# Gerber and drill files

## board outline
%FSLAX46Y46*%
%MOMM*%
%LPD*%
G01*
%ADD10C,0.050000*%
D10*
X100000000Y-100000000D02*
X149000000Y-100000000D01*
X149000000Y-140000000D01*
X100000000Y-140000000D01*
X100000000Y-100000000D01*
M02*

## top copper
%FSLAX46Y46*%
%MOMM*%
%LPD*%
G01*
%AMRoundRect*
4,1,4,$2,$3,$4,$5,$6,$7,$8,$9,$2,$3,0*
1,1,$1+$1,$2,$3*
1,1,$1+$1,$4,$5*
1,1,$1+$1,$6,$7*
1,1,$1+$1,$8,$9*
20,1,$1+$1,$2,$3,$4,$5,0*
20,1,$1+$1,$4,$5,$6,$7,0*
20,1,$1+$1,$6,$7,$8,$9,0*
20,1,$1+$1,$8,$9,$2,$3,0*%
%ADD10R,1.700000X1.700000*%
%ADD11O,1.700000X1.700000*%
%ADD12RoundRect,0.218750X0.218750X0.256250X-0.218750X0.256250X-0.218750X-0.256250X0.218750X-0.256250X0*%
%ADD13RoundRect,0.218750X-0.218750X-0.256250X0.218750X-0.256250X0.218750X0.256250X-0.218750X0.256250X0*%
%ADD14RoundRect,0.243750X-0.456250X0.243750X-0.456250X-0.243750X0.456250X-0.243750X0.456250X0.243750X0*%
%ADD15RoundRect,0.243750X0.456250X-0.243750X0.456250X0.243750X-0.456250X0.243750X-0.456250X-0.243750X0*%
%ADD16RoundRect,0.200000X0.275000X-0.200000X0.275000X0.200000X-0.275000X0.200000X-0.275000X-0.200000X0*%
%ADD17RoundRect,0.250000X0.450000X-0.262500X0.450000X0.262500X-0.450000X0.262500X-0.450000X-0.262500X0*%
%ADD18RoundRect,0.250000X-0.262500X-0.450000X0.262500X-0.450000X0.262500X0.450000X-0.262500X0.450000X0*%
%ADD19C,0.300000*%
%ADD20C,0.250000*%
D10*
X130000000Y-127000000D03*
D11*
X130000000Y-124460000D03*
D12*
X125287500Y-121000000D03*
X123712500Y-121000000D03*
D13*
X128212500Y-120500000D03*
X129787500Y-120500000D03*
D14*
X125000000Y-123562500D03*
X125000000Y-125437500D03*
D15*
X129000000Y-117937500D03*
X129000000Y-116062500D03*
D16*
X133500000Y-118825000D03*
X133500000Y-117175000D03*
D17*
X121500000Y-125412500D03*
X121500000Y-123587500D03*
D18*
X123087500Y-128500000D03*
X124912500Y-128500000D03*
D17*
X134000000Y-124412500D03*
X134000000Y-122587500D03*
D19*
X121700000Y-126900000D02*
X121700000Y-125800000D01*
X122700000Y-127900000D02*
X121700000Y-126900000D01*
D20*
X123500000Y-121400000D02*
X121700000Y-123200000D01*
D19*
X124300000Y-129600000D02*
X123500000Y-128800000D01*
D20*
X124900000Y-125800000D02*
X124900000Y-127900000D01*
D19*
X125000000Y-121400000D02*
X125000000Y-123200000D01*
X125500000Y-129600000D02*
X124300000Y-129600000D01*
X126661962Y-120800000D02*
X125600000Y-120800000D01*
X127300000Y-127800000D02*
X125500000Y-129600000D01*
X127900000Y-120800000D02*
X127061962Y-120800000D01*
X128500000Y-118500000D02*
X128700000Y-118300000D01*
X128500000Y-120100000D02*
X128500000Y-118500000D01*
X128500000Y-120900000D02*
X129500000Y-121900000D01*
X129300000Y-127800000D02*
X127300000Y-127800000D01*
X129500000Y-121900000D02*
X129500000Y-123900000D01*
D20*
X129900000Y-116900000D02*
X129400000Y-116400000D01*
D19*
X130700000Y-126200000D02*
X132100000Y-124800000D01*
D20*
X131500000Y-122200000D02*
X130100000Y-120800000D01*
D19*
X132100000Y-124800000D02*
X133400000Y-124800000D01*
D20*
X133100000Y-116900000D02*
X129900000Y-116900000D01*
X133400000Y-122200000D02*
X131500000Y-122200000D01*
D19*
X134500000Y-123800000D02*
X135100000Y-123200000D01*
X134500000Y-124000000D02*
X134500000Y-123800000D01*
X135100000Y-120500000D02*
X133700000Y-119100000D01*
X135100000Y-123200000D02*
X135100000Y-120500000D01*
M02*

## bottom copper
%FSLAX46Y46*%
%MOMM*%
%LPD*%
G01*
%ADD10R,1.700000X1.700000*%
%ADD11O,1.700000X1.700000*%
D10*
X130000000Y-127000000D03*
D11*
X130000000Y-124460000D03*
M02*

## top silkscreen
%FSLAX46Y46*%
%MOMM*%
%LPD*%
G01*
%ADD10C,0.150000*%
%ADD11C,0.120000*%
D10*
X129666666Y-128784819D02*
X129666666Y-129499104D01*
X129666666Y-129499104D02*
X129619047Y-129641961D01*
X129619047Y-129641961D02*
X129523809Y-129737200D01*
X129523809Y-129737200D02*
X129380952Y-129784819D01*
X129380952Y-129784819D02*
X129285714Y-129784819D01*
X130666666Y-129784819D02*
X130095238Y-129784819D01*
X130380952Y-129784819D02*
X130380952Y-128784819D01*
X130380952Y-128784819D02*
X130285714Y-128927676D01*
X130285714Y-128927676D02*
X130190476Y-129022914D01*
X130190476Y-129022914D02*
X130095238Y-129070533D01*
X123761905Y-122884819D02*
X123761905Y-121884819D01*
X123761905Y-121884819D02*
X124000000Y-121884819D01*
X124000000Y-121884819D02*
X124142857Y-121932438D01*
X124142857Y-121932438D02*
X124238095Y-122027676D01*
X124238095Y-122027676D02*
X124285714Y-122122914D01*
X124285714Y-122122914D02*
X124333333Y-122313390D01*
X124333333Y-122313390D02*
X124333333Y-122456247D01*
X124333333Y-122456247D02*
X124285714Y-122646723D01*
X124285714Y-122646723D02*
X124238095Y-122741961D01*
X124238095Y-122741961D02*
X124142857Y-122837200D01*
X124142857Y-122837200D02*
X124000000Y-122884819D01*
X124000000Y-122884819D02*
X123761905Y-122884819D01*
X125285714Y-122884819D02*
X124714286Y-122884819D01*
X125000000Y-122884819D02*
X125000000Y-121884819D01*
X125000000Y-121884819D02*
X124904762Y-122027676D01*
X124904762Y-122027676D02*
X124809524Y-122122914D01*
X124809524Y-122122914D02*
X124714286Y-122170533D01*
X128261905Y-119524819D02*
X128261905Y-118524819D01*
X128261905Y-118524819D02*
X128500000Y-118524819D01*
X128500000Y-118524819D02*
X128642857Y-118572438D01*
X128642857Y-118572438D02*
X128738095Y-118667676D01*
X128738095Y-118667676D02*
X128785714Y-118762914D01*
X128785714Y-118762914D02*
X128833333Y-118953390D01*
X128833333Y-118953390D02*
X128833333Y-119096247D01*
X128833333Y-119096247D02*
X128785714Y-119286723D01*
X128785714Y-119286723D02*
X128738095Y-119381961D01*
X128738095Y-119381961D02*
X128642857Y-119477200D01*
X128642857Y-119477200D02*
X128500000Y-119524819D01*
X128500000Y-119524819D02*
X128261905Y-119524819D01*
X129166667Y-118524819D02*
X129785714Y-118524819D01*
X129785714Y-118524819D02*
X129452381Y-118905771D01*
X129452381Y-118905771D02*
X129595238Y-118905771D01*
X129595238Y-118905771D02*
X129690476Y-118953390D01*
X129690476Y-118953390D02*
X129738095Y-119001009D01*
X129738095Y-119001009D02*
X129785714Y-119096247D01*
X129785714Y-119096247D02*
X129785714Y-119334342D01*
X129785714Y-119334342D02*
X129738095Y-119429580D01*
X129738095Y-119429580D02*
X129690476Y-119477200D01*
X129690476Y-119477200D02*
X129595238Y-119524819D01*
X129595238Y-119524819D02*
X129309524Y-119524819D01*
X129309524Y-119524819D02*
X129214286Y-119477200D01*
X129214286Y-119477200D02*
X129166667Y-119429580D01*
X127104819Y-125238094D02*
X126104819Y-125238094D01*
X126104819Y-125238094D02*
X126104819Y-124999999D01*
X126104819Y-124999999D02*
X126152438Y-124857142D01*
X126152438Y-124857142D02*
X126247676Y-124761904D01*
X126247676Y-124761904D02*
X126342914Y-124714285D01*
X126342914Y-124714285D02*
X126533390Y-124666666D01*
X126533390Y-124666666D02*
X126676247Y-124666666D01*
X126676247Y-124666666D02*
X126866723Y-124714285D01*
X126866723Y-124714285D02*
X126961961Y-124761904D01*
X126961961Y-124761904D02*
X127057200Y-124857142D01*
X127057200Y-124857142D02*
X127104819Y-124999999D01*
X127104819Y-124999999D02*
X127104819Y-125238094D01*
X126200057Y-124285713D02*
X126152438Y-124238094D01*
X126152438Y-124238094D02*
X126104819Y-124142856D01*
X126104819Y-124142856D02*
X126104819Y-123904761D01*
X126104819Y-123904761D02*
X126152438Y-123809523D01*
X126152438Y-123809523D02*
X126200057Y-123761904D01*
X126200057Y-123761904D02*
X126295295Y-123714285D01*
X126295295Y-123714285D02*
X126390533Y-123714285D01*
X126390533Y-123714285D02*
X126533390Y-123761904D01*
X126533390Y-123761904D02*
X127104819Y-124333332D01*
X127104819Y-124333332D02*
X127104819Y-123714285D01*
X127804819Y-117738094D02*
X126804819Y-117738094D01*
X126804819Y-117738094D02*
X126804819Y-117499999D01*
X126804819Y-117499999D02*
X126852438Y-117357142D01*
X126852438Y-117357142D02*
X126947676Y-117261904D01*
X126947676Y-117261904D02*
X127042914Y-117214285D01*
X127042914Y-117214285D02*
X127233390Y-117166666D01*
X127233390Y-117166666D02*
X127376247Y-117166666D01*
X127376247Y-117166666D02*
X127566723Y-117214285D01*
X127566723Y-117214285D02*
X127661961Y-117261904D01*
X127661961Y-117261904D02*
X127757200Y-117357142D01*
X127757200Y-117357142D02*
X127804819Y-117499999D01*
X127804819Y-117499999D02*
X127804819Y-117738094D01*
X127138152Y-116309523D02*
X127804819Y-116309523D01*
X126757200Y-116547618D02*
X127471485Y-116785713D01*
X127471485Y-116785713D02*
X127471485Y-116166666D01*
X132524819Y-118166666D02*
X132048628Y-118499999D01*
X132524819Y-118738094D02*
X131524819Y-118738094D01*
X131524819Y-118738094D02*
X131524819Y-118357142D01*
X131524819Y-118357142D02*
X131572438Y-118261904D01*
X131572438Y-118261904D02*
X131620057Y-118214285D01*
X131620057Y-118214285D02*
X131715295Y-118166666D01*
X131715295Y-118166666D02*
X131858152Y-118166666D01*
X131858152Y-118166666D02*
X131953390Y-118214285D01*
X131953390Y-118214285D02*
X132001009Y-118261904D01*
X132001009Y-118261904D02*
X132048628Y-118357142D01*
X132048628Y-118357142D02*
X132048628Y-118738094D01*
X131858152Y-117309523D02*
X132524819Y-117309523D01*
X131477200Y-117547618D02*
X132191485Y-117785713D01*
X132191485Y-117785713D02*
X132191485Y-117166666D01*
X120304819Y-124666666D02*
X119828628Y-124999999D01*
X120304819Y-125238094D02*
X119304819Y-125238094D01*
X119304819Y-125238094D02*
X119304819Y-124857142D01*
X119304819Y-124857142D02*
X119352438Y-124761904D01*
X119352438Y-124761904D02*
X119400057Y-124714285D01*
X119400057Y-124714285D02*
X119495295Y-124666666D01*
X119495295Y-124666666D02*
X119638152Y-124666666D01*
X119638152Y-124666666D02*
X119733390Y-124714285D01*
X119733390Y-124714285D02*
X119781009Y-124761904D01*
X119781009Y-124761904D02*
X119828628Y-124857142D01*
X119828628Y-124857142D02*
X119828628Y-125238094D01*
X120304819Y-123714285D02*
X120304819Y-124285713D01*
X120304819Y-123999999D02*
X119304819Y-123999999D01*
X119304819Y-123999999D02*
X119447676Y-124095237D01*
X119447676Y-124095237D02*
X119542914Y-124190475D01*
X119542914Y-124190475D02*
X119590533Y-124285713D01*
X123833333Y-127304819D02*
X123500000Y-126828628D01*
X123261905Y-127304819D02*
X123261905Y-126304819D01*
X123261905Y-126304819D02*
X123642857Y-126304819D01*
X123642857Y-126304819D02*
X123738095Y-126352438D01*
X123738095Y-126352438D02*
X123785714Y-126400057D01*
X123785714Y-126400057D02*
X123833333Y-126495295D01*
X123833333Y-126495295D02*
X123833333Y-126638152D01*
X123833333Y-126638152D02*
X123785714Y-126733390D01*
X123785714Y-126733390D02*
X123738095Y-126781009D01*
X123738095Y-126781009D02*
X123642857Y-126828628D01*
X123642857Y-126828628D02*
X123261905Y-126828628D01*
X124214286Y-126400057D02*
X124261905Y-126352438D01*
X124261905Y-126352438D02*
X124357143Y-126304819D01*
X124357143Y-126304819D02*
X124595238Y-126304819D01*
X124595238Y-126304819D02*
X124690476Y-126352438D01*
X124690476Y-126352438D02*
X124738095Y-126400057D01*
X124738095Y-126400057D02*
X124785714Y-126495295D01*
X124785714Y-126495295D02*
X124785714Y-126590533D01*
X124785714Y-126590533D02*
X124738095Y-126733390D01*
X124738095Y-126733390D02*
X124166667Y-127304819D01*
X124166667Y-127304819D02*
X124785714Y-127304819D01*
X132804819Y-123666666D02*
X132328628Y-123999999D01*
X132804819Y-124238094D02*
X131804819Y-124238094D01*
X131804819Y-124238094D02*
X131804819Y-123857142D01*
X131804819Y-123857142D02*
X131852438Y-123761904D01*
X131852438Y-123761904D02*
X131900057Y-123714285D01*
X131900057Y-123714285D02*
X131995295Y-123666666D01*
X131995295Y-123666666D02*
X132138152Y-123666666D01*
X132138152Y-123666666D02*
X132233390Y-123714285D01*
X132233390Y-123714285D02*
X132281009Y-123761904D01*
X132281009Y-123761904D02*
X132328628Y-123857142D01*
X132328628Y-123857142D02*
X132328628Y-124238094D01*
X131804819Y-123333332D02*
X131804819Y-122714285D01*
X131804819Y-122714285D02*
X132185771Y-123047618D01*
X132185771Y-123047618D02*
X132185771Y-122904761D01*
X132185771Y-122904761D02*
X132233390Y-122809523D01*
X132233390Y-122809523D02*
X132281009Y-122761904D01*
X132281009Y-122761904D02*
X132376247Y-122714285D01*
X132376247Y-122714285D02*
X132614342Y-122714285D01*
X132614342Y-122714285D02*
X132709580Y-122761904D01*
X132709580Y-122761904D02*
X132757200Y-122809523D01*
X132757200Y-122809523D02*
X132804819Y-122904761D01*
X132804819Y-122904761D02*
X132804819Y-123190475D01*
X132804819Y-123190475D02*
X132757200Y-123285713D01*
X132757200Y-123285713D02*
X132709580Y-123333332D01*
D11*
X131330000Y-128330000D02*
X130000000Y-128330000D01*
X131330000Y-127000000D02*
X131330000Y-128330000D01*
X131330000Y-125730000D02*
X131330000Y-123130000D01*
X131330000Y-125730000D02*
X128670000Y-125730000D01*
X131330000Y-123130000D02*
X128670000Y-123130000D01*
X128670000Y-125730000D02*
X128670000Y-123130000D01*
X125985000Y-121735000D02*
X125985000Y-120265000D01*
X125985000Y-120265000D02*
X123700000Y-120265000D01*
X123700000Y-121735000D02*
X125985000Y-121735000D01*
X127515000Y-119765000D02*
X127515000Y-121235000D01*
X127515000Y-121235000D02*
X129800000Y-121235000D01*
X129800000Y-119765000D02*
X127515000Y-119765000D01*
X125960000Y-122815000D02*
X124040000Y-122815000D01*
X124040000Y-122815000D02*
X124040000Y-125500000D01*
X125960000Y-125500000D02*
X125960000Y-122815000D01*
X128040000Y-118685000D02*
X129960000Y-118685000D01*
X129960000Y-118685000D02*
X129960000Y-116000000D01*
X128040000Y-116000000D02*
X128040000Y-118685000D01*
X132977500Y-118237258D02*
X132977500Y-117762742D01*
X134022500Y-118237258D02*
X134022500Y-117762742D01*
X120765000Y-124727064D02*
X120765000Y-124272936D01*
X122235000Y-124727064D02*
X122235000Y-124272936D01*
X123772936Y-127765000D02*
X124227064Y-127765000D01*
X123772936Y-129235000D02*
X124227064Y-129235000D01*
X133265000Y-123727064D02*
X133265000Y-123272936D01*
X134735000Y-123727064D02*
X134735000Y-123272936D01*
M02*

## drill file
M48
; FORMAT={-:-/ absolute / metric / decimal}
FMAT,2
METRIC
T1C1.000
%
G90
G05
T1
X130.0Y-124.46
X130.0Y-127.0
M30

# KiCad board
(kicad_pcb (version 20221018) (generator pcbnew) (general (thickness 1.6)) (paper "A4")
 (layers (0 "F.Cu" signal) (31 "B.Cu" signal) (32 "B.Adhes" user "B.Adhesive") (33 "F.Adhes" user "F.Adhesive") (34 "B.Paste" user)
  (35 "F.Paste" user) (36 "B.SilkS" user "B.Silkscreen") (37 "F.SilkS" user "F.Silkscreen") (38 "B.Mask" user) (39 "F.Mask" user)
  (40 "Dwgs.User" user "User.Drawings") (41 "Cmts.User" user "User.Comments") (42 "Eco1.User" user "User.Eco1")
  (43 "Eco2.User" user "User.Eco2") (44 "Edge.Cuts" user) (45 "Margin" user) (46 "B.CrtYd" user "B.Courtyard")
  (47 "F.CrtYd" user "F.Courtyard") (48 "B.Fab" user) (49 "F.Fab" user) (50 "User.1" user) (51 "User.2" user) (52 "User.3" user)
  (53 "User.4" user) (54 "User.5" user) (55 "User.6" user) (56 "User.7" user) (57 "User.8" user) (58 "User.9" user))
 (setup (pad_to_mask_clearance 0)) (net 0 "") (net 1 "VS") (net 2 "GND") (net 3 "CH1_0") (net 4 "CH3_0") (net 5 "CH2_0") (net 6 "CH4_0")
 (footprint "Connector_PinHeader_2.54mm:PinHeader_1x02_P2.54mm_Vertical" (layer "F.Cu") (at 130 127 180)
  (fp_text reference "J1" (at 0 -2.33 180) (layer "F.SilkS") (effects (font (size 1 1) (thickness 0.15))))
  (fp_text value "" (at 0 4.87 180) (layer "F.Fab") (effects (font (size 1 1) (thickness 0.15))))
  (fp_line (start -1.33 -1.33) (end 0 -1.33) (stroke (width 0.12) (type solid)) (layer "F.SilkS"))
  (fp_line (start -1.33 0) (end -1.33 -1.33) (stroke (width 0.12) (type solid)) (layer "F.SilkS"))
  (fp_line (start -1.33 1.27) (end -1.33 3.87) (stroke (width 0.12) (type solid)) (layer "F.SilkS"))
  (fp_line (start -1.33 1.27) (end 1.33 1.27) (stroke (width 0.12) (type solid)) (layer "F.SilkS"))
  (fp_line (start -1.33 3.87) (end 1.33 3.87) (stroke (width 0.12) (type solid)) (layer "F.SilkS"))
  (fp_line (start 1.33 1.27) (end 1.33 3.87) (stroke (width 0.12) (type solid)) (layer "F.SilkS"))
  (pad "1" thru_hole rect (at 0 0 180) (size 1.7 1.7) (drill 1) (layers "*.Cu" "*.Mask") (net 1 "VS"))
  (pad "2" thru_hole oval (at 0 2.54 180) (size 1.7 1.7) (drill 1) (layers "*.Cu" "*.Mask") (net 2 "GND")))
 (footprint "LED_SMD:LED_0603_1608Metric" (layer "F.Cu") (at 124.5 121 180)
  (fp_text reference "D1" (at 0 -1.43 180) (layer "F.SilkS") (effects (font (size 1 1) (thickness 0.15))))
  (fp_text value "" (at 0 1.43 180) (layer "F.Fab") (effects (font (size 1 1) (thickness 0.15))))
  (fp_line (start -1.485 -0.735) (end -1.485 0.735) (stroke (width 0.12) (type solid)) (layer "F.SilkS"))
  (fp_line (start -1.485 0.735) (end 0.8 0.735) (stroke (width 0.12) (type solid)) (layer "F.SilkS"))
  (fp_line (start 0.8 -0.735) (end -1.485 -0.735) (stroke (width 0.12) (type solid)) (layer "F.SilkS"))
  (pad "1" smd roundrect (at -0.7875 0 180) (size 0.875 0.95) (layers "F.Cu" "F.Paste" "F.Mask") (roundrect_rratio 0.25) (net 2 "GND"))
  (pad "2" smd roundrect (at 0.7875 0 180) (size 0.875 0.95) (layers "F.Cu" "F.Paste" "F.Mask") (roundrect_rratio 0.25) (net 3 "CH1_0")))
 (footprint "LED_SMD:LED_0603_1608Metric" (layer "F.Cu") (at 129 120.5)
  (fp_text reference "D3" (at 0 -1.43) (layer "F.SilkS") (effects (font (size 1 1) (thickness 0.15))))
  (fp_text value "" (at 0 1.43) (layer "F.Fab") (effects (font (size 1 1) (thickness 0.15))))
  (fp_line (start -1.485 -0.735) (end -1.485 0.735) (stroke (width 0.12) (type solid)) (layer "F.SilkS"))
  (fp_line (start -1.485 0.735) (end 0.8 0.735) (stroke (width 0.12) (type solid)) (layer "F.SilkS"))
  (fp_line (start 0.8 -0.735) (end -1.485 -0.735) (stroke (width 0.12) (type solid)) (layer "F.SilkS"))
  (pad "1" smd roundrect (at -0.7875 0) (size 0.875 0.95) (layers "F.Cu" "F.Paste" "F.Mask") (roundrect_rratio 0.25) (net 2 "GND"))
  (pad "2" smd roundrect (at 0.7875 0) (size 0.875 0.95) (layers "F.Cu" "F.Paste" "F.Mask") (roundrect_rratio 0.25) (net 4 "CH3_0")))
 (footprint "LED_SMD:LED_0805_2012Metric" (layer "F.Cu") (at 125 124.5 -90)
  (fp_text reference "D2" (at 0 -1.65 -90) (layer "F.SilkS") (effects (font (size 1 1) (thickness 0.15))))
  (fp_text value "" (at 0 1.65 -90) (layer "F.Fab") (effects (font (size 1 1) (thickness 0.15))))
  (fp_line (start -1.685 -0.96) (end -1.685 0.96) (stroke (width 0.12) (type solid)) (layer "F.SilkS"))
  (fp_line (start -1.685 0.96) (end 1 0.96) (stroke (width 0.12) (type solid)) (layer "F.SilkS"))
  (fp_line (start 1 -0.96) (end -1.685 -0.96) (stroke (width 0.12) (type solid)) (layer "F.SilkS"))
  (pad "1" smd roundrect (at -0.9375 0 270) (size 0.975 1.4) (layers "F.Cu" "F.Paste" "F.Mask") (roundrect_rratio 0.25) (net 2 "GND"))
  (pad "2" smd roundrect (at 0.9375 0 270) (size 0.975 1.4) (layers "F.Cu" "F.Paste" "F.Mask") (roundrect_rratio 0.25) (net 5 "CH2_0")))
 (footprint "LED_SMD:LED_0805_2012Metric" (layer "F.Cu") (at 129 117 90)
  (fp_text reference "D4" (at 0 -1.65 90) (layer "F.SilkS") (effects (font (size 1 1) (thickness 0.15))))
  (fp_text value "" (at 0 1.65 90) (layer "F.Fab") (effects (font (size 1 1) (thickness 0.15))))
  (fp_line (start -1.685 -0.96) (end -1.685 0.96) (stroke (width 0.12) (type solid)) (layer "F.SilkS"))
  (fp_line (start -1.685 0.96) (end 1 0.96) (stroke (width 0.12) (type solid)) (layer "F.SilkS"))
  (fp_line (start 1 -0.96) (end -1.685 -0.96) (stroke (width 0.12) (type solid)) (layer "F.SilkS"))
  (pad "1" smd roundrect (at -0.9375 0 90) (size 0.975 1.4) (layers "F.Cu" "F.Paste" "F.Mask") (roundrect_rratio 0.25) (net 2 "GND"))
  (pad "2" smd roundrect (at 0.9375 0 90) (size 0.975 1.4) (layers "F.Cu" "F.Paste" "F.Mask") (roundrect_rratio 0.25) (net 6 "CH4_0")))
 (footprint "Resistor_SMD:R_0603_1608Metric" (layer "F.Cu") (at 133.5 118 90)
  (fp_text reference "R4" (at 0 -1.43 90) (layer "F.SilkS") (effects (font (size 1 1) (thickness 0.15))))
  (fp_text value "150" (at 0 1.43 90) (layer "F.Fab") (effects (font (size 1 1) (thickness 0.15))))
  (fp_line (start -0.237258 -0.5225) (end 0.237258 -0.5225) (stroke (width 0.12) (type solid)) (layer "F.SilkS"))
  (fp_line (start -0.237258 0.5225) (end 0.237258 0.5225) (stroke (width 0.12) (type solid)) (layer "F.SilkS"))
  (pad "1" smd roundrect (at -0.825 0 90) (size 0.8 0.95) (layers "F.Cu" "F.Paste" "F.Mask") (roundrect_rratio 0.25) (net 1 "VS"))
  (pad "2" smd roundrect (at 0.825 0 90) (size 0.8 0.95) (layers "F.Cu" "F.Paste" "F.Mask") (roundrect_rratio 0.25) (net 6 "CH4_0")))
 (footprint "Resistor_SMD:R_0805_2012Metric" (layer "F.Cu") (at 121.5 124.5 90)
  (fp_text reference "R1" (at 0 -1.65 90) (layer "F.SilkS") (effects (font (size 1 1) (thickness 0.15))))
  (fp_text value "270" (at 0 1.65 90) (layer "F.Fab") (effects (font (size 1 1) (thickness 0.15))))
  (fp_line (start -0.227064 -0.735) (end 0.227064 -0.735) (stroke (width 0.12) (type solid)) (layer "F.SilkS"))
  (fp_line (start -0.227064 0.735) (end 0.227064 0.735) (stroke (width 0.12) (type solid)) (layer "F.SilkS"))
  (pad "1" smd roundrect (at -0.9125 0 90) (size 1.025 1.4) (layers "F.Cu" "F.Paste" "F.Mask") (roundrect_rratio 0.243902) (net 1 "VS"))
  (pad "2" smd roundrect (at 0.9125 0 90) (size 1.025 1.4) (layers "F.Cu" "F.Paste" "F.Mask") (roundrect_rratio 0.243902) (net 3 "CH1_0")))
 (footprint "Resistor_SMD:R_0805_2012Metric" (layer "F.Cu") (at 124 128.5)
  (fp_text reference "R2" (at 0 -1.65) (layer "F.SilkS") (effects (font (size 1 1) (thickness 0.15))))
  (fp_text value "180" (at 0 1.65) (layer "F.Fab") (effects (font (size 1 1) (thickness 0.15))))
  (fp_line (start -0.227064 -0.735) (end 0.227064 -0.735) (stroke (width 0.12) (type solid)) (layer "F.SilkS"))
  (fp_line (start -0.227064 0.735) (end 0.227064 0.735) (stroke (width 0.12) (type solid)) (layer "F.SilkS"))
  (pad "1" smd roundrect (at -0.9125 0) (size 1.025 1.4) (layers "F.Cu" "F.Paste" "F.Mask") (roundrect_rratio 0.243902) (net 1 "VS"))
  (pad "2" smd roundrect (at 0.9125 0) (size 1.025 1.4) (layers "F.Cu" "F.Paste" "F.Mask") (roundrect_rratio 0.243902) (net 5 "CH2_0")))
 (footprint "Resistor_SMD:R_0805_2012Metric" (layer "F.Cu") (at 134 123.5 90)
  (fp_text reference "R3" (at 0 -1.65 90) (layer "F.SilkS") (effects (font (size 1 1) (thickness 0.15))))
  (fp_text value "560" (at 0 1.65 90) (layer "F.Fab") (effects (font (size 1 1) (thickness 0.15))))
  (fp_line (start -0.227064 -0.735) (end 0.227064 -0.735) (stroke (width 0.12) (type solid)) (layer "F.SilkS"))
  (fp_line (start -0.227064 0.735) (end 0.227064 0.735) (stroke (width 0.12) (type solid)) (layer "F.SilkS"))
  (pad "1" smd roundrect (at -0.9125 0 90) (size 1.025 1.4) (layers "F.Cu" "F.Paste" "F.Mask") (roundrect_rratio 0.243902) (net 1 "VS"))
  (pad "2" smd roundrect (at 0.9125 0 90) (size 1.025 1.4) (layers "F.Cu" "F.Paste" "F.Mask") (roundrect_rratio 0.243902) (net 4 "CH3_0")))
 (gr_rect (start 100 100) (end 149 140) (stroke (width 0.05) (type default)) (fill none) (layer "Edge.Cuts"))
 (segment (start 121.7 126.9) (end 121.7 125.8) (width 0.3) (layer "F.Cu") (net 1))
 (segment (start 122.7 127.9) (end 121.7 126.9) (width 0.3) (layer "F.Cu") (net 1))
 (segment (start 123.5 121.4) (end 121.7 123.2) (width 0.25) (layer "F.Cu") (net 3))
 (segment (start 124.3 129.6) (end 123.5 128.8) (width 0.3) (layer "F.Cu") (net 1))
 (segment (start 124.9 125.8) (end 124.9 127.9) (width 0.25) (layer "F.Cu") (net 5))
 (segment (start 125 121.4) (end 125 123.2) (width 0.3) (layer "F.Cu") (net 2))
 (segment (start 125.5 129.6) (end 124.3 129.6) (width 0.3) (layer "F.Cu") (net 1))
 (segment (start 126.661962 120.8) (end 125.6 120.8) (width 0.3) (layer "F.Cu") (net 2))
 (segment (start 127.3 127.8) (end 125.5 129.6) (width 0.3) (layer "F.Cu") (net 1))
 (segment (start 127.9 120.8) (end 127.061962 120.8) (width 0.3) (layer "F.Cu") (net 2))
 (segment (start 128.5 118.5) (end 128.7 118.3) (width 0.3) (layer "F.Cu") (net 2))
 (segment (start 128.5 120.1) (end 128.5 118.5) (width 0.3) (layer "F.Cu") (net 2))
 (segment (start 128.5 120.9) (end 129.5 121.9) (width 0.3) (layer "F.Cu") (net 2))
 (segment (start 129.3 127.8) (end 127.3 127.8) (width 0.3) (layer "F.Cu") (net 1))
 (segment (start 129.5 121.9) (end 129.5 123.9) (width 0.3) (layer "F.Cu") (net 2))
 (segment (start 129.9 116.9) (end 129.4 116.4) (width 0.25) (layer "F.Cu") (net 6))
 (segment (start 130.7 126.2) (end 132.1 124.8) (width 0.3) (layer "F.Cu") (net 1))
 (segment (start 131.5 122.2) (end 130.1 120.8) (width 0.25) (layer "F.Cu") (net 4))
 (segment (start 132.1 124.8) (end 133.4 124.8) (width 0.3) (layer "F.Cu") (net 1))
 (segment (start 133.1 116.9) (end 129.9 116.9) (width 0.25) (layer "F.Cu") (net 6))
 (segment (start 133.4 122.2) (end 131.5 122.2) (width 0.25) (layer "F.Cu") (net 4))
 (segment (start 134.5 123.8) (end 135.1 123.2) (width 0.3) (layer "F.Cu") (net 1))
 (segment (start 134.5 124) (end 134.5 123.8) (width 0.3) (layer "F.Cu") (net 1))
 (segment (start 135.1 120.5) (end 133.7 119.1) (width 0.3) (layer "F.Cu") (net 1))
 (segment (start 135.1 123.2) (end 135.1 120.5) (width 0.3) (layer "F.Cu") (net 1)))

